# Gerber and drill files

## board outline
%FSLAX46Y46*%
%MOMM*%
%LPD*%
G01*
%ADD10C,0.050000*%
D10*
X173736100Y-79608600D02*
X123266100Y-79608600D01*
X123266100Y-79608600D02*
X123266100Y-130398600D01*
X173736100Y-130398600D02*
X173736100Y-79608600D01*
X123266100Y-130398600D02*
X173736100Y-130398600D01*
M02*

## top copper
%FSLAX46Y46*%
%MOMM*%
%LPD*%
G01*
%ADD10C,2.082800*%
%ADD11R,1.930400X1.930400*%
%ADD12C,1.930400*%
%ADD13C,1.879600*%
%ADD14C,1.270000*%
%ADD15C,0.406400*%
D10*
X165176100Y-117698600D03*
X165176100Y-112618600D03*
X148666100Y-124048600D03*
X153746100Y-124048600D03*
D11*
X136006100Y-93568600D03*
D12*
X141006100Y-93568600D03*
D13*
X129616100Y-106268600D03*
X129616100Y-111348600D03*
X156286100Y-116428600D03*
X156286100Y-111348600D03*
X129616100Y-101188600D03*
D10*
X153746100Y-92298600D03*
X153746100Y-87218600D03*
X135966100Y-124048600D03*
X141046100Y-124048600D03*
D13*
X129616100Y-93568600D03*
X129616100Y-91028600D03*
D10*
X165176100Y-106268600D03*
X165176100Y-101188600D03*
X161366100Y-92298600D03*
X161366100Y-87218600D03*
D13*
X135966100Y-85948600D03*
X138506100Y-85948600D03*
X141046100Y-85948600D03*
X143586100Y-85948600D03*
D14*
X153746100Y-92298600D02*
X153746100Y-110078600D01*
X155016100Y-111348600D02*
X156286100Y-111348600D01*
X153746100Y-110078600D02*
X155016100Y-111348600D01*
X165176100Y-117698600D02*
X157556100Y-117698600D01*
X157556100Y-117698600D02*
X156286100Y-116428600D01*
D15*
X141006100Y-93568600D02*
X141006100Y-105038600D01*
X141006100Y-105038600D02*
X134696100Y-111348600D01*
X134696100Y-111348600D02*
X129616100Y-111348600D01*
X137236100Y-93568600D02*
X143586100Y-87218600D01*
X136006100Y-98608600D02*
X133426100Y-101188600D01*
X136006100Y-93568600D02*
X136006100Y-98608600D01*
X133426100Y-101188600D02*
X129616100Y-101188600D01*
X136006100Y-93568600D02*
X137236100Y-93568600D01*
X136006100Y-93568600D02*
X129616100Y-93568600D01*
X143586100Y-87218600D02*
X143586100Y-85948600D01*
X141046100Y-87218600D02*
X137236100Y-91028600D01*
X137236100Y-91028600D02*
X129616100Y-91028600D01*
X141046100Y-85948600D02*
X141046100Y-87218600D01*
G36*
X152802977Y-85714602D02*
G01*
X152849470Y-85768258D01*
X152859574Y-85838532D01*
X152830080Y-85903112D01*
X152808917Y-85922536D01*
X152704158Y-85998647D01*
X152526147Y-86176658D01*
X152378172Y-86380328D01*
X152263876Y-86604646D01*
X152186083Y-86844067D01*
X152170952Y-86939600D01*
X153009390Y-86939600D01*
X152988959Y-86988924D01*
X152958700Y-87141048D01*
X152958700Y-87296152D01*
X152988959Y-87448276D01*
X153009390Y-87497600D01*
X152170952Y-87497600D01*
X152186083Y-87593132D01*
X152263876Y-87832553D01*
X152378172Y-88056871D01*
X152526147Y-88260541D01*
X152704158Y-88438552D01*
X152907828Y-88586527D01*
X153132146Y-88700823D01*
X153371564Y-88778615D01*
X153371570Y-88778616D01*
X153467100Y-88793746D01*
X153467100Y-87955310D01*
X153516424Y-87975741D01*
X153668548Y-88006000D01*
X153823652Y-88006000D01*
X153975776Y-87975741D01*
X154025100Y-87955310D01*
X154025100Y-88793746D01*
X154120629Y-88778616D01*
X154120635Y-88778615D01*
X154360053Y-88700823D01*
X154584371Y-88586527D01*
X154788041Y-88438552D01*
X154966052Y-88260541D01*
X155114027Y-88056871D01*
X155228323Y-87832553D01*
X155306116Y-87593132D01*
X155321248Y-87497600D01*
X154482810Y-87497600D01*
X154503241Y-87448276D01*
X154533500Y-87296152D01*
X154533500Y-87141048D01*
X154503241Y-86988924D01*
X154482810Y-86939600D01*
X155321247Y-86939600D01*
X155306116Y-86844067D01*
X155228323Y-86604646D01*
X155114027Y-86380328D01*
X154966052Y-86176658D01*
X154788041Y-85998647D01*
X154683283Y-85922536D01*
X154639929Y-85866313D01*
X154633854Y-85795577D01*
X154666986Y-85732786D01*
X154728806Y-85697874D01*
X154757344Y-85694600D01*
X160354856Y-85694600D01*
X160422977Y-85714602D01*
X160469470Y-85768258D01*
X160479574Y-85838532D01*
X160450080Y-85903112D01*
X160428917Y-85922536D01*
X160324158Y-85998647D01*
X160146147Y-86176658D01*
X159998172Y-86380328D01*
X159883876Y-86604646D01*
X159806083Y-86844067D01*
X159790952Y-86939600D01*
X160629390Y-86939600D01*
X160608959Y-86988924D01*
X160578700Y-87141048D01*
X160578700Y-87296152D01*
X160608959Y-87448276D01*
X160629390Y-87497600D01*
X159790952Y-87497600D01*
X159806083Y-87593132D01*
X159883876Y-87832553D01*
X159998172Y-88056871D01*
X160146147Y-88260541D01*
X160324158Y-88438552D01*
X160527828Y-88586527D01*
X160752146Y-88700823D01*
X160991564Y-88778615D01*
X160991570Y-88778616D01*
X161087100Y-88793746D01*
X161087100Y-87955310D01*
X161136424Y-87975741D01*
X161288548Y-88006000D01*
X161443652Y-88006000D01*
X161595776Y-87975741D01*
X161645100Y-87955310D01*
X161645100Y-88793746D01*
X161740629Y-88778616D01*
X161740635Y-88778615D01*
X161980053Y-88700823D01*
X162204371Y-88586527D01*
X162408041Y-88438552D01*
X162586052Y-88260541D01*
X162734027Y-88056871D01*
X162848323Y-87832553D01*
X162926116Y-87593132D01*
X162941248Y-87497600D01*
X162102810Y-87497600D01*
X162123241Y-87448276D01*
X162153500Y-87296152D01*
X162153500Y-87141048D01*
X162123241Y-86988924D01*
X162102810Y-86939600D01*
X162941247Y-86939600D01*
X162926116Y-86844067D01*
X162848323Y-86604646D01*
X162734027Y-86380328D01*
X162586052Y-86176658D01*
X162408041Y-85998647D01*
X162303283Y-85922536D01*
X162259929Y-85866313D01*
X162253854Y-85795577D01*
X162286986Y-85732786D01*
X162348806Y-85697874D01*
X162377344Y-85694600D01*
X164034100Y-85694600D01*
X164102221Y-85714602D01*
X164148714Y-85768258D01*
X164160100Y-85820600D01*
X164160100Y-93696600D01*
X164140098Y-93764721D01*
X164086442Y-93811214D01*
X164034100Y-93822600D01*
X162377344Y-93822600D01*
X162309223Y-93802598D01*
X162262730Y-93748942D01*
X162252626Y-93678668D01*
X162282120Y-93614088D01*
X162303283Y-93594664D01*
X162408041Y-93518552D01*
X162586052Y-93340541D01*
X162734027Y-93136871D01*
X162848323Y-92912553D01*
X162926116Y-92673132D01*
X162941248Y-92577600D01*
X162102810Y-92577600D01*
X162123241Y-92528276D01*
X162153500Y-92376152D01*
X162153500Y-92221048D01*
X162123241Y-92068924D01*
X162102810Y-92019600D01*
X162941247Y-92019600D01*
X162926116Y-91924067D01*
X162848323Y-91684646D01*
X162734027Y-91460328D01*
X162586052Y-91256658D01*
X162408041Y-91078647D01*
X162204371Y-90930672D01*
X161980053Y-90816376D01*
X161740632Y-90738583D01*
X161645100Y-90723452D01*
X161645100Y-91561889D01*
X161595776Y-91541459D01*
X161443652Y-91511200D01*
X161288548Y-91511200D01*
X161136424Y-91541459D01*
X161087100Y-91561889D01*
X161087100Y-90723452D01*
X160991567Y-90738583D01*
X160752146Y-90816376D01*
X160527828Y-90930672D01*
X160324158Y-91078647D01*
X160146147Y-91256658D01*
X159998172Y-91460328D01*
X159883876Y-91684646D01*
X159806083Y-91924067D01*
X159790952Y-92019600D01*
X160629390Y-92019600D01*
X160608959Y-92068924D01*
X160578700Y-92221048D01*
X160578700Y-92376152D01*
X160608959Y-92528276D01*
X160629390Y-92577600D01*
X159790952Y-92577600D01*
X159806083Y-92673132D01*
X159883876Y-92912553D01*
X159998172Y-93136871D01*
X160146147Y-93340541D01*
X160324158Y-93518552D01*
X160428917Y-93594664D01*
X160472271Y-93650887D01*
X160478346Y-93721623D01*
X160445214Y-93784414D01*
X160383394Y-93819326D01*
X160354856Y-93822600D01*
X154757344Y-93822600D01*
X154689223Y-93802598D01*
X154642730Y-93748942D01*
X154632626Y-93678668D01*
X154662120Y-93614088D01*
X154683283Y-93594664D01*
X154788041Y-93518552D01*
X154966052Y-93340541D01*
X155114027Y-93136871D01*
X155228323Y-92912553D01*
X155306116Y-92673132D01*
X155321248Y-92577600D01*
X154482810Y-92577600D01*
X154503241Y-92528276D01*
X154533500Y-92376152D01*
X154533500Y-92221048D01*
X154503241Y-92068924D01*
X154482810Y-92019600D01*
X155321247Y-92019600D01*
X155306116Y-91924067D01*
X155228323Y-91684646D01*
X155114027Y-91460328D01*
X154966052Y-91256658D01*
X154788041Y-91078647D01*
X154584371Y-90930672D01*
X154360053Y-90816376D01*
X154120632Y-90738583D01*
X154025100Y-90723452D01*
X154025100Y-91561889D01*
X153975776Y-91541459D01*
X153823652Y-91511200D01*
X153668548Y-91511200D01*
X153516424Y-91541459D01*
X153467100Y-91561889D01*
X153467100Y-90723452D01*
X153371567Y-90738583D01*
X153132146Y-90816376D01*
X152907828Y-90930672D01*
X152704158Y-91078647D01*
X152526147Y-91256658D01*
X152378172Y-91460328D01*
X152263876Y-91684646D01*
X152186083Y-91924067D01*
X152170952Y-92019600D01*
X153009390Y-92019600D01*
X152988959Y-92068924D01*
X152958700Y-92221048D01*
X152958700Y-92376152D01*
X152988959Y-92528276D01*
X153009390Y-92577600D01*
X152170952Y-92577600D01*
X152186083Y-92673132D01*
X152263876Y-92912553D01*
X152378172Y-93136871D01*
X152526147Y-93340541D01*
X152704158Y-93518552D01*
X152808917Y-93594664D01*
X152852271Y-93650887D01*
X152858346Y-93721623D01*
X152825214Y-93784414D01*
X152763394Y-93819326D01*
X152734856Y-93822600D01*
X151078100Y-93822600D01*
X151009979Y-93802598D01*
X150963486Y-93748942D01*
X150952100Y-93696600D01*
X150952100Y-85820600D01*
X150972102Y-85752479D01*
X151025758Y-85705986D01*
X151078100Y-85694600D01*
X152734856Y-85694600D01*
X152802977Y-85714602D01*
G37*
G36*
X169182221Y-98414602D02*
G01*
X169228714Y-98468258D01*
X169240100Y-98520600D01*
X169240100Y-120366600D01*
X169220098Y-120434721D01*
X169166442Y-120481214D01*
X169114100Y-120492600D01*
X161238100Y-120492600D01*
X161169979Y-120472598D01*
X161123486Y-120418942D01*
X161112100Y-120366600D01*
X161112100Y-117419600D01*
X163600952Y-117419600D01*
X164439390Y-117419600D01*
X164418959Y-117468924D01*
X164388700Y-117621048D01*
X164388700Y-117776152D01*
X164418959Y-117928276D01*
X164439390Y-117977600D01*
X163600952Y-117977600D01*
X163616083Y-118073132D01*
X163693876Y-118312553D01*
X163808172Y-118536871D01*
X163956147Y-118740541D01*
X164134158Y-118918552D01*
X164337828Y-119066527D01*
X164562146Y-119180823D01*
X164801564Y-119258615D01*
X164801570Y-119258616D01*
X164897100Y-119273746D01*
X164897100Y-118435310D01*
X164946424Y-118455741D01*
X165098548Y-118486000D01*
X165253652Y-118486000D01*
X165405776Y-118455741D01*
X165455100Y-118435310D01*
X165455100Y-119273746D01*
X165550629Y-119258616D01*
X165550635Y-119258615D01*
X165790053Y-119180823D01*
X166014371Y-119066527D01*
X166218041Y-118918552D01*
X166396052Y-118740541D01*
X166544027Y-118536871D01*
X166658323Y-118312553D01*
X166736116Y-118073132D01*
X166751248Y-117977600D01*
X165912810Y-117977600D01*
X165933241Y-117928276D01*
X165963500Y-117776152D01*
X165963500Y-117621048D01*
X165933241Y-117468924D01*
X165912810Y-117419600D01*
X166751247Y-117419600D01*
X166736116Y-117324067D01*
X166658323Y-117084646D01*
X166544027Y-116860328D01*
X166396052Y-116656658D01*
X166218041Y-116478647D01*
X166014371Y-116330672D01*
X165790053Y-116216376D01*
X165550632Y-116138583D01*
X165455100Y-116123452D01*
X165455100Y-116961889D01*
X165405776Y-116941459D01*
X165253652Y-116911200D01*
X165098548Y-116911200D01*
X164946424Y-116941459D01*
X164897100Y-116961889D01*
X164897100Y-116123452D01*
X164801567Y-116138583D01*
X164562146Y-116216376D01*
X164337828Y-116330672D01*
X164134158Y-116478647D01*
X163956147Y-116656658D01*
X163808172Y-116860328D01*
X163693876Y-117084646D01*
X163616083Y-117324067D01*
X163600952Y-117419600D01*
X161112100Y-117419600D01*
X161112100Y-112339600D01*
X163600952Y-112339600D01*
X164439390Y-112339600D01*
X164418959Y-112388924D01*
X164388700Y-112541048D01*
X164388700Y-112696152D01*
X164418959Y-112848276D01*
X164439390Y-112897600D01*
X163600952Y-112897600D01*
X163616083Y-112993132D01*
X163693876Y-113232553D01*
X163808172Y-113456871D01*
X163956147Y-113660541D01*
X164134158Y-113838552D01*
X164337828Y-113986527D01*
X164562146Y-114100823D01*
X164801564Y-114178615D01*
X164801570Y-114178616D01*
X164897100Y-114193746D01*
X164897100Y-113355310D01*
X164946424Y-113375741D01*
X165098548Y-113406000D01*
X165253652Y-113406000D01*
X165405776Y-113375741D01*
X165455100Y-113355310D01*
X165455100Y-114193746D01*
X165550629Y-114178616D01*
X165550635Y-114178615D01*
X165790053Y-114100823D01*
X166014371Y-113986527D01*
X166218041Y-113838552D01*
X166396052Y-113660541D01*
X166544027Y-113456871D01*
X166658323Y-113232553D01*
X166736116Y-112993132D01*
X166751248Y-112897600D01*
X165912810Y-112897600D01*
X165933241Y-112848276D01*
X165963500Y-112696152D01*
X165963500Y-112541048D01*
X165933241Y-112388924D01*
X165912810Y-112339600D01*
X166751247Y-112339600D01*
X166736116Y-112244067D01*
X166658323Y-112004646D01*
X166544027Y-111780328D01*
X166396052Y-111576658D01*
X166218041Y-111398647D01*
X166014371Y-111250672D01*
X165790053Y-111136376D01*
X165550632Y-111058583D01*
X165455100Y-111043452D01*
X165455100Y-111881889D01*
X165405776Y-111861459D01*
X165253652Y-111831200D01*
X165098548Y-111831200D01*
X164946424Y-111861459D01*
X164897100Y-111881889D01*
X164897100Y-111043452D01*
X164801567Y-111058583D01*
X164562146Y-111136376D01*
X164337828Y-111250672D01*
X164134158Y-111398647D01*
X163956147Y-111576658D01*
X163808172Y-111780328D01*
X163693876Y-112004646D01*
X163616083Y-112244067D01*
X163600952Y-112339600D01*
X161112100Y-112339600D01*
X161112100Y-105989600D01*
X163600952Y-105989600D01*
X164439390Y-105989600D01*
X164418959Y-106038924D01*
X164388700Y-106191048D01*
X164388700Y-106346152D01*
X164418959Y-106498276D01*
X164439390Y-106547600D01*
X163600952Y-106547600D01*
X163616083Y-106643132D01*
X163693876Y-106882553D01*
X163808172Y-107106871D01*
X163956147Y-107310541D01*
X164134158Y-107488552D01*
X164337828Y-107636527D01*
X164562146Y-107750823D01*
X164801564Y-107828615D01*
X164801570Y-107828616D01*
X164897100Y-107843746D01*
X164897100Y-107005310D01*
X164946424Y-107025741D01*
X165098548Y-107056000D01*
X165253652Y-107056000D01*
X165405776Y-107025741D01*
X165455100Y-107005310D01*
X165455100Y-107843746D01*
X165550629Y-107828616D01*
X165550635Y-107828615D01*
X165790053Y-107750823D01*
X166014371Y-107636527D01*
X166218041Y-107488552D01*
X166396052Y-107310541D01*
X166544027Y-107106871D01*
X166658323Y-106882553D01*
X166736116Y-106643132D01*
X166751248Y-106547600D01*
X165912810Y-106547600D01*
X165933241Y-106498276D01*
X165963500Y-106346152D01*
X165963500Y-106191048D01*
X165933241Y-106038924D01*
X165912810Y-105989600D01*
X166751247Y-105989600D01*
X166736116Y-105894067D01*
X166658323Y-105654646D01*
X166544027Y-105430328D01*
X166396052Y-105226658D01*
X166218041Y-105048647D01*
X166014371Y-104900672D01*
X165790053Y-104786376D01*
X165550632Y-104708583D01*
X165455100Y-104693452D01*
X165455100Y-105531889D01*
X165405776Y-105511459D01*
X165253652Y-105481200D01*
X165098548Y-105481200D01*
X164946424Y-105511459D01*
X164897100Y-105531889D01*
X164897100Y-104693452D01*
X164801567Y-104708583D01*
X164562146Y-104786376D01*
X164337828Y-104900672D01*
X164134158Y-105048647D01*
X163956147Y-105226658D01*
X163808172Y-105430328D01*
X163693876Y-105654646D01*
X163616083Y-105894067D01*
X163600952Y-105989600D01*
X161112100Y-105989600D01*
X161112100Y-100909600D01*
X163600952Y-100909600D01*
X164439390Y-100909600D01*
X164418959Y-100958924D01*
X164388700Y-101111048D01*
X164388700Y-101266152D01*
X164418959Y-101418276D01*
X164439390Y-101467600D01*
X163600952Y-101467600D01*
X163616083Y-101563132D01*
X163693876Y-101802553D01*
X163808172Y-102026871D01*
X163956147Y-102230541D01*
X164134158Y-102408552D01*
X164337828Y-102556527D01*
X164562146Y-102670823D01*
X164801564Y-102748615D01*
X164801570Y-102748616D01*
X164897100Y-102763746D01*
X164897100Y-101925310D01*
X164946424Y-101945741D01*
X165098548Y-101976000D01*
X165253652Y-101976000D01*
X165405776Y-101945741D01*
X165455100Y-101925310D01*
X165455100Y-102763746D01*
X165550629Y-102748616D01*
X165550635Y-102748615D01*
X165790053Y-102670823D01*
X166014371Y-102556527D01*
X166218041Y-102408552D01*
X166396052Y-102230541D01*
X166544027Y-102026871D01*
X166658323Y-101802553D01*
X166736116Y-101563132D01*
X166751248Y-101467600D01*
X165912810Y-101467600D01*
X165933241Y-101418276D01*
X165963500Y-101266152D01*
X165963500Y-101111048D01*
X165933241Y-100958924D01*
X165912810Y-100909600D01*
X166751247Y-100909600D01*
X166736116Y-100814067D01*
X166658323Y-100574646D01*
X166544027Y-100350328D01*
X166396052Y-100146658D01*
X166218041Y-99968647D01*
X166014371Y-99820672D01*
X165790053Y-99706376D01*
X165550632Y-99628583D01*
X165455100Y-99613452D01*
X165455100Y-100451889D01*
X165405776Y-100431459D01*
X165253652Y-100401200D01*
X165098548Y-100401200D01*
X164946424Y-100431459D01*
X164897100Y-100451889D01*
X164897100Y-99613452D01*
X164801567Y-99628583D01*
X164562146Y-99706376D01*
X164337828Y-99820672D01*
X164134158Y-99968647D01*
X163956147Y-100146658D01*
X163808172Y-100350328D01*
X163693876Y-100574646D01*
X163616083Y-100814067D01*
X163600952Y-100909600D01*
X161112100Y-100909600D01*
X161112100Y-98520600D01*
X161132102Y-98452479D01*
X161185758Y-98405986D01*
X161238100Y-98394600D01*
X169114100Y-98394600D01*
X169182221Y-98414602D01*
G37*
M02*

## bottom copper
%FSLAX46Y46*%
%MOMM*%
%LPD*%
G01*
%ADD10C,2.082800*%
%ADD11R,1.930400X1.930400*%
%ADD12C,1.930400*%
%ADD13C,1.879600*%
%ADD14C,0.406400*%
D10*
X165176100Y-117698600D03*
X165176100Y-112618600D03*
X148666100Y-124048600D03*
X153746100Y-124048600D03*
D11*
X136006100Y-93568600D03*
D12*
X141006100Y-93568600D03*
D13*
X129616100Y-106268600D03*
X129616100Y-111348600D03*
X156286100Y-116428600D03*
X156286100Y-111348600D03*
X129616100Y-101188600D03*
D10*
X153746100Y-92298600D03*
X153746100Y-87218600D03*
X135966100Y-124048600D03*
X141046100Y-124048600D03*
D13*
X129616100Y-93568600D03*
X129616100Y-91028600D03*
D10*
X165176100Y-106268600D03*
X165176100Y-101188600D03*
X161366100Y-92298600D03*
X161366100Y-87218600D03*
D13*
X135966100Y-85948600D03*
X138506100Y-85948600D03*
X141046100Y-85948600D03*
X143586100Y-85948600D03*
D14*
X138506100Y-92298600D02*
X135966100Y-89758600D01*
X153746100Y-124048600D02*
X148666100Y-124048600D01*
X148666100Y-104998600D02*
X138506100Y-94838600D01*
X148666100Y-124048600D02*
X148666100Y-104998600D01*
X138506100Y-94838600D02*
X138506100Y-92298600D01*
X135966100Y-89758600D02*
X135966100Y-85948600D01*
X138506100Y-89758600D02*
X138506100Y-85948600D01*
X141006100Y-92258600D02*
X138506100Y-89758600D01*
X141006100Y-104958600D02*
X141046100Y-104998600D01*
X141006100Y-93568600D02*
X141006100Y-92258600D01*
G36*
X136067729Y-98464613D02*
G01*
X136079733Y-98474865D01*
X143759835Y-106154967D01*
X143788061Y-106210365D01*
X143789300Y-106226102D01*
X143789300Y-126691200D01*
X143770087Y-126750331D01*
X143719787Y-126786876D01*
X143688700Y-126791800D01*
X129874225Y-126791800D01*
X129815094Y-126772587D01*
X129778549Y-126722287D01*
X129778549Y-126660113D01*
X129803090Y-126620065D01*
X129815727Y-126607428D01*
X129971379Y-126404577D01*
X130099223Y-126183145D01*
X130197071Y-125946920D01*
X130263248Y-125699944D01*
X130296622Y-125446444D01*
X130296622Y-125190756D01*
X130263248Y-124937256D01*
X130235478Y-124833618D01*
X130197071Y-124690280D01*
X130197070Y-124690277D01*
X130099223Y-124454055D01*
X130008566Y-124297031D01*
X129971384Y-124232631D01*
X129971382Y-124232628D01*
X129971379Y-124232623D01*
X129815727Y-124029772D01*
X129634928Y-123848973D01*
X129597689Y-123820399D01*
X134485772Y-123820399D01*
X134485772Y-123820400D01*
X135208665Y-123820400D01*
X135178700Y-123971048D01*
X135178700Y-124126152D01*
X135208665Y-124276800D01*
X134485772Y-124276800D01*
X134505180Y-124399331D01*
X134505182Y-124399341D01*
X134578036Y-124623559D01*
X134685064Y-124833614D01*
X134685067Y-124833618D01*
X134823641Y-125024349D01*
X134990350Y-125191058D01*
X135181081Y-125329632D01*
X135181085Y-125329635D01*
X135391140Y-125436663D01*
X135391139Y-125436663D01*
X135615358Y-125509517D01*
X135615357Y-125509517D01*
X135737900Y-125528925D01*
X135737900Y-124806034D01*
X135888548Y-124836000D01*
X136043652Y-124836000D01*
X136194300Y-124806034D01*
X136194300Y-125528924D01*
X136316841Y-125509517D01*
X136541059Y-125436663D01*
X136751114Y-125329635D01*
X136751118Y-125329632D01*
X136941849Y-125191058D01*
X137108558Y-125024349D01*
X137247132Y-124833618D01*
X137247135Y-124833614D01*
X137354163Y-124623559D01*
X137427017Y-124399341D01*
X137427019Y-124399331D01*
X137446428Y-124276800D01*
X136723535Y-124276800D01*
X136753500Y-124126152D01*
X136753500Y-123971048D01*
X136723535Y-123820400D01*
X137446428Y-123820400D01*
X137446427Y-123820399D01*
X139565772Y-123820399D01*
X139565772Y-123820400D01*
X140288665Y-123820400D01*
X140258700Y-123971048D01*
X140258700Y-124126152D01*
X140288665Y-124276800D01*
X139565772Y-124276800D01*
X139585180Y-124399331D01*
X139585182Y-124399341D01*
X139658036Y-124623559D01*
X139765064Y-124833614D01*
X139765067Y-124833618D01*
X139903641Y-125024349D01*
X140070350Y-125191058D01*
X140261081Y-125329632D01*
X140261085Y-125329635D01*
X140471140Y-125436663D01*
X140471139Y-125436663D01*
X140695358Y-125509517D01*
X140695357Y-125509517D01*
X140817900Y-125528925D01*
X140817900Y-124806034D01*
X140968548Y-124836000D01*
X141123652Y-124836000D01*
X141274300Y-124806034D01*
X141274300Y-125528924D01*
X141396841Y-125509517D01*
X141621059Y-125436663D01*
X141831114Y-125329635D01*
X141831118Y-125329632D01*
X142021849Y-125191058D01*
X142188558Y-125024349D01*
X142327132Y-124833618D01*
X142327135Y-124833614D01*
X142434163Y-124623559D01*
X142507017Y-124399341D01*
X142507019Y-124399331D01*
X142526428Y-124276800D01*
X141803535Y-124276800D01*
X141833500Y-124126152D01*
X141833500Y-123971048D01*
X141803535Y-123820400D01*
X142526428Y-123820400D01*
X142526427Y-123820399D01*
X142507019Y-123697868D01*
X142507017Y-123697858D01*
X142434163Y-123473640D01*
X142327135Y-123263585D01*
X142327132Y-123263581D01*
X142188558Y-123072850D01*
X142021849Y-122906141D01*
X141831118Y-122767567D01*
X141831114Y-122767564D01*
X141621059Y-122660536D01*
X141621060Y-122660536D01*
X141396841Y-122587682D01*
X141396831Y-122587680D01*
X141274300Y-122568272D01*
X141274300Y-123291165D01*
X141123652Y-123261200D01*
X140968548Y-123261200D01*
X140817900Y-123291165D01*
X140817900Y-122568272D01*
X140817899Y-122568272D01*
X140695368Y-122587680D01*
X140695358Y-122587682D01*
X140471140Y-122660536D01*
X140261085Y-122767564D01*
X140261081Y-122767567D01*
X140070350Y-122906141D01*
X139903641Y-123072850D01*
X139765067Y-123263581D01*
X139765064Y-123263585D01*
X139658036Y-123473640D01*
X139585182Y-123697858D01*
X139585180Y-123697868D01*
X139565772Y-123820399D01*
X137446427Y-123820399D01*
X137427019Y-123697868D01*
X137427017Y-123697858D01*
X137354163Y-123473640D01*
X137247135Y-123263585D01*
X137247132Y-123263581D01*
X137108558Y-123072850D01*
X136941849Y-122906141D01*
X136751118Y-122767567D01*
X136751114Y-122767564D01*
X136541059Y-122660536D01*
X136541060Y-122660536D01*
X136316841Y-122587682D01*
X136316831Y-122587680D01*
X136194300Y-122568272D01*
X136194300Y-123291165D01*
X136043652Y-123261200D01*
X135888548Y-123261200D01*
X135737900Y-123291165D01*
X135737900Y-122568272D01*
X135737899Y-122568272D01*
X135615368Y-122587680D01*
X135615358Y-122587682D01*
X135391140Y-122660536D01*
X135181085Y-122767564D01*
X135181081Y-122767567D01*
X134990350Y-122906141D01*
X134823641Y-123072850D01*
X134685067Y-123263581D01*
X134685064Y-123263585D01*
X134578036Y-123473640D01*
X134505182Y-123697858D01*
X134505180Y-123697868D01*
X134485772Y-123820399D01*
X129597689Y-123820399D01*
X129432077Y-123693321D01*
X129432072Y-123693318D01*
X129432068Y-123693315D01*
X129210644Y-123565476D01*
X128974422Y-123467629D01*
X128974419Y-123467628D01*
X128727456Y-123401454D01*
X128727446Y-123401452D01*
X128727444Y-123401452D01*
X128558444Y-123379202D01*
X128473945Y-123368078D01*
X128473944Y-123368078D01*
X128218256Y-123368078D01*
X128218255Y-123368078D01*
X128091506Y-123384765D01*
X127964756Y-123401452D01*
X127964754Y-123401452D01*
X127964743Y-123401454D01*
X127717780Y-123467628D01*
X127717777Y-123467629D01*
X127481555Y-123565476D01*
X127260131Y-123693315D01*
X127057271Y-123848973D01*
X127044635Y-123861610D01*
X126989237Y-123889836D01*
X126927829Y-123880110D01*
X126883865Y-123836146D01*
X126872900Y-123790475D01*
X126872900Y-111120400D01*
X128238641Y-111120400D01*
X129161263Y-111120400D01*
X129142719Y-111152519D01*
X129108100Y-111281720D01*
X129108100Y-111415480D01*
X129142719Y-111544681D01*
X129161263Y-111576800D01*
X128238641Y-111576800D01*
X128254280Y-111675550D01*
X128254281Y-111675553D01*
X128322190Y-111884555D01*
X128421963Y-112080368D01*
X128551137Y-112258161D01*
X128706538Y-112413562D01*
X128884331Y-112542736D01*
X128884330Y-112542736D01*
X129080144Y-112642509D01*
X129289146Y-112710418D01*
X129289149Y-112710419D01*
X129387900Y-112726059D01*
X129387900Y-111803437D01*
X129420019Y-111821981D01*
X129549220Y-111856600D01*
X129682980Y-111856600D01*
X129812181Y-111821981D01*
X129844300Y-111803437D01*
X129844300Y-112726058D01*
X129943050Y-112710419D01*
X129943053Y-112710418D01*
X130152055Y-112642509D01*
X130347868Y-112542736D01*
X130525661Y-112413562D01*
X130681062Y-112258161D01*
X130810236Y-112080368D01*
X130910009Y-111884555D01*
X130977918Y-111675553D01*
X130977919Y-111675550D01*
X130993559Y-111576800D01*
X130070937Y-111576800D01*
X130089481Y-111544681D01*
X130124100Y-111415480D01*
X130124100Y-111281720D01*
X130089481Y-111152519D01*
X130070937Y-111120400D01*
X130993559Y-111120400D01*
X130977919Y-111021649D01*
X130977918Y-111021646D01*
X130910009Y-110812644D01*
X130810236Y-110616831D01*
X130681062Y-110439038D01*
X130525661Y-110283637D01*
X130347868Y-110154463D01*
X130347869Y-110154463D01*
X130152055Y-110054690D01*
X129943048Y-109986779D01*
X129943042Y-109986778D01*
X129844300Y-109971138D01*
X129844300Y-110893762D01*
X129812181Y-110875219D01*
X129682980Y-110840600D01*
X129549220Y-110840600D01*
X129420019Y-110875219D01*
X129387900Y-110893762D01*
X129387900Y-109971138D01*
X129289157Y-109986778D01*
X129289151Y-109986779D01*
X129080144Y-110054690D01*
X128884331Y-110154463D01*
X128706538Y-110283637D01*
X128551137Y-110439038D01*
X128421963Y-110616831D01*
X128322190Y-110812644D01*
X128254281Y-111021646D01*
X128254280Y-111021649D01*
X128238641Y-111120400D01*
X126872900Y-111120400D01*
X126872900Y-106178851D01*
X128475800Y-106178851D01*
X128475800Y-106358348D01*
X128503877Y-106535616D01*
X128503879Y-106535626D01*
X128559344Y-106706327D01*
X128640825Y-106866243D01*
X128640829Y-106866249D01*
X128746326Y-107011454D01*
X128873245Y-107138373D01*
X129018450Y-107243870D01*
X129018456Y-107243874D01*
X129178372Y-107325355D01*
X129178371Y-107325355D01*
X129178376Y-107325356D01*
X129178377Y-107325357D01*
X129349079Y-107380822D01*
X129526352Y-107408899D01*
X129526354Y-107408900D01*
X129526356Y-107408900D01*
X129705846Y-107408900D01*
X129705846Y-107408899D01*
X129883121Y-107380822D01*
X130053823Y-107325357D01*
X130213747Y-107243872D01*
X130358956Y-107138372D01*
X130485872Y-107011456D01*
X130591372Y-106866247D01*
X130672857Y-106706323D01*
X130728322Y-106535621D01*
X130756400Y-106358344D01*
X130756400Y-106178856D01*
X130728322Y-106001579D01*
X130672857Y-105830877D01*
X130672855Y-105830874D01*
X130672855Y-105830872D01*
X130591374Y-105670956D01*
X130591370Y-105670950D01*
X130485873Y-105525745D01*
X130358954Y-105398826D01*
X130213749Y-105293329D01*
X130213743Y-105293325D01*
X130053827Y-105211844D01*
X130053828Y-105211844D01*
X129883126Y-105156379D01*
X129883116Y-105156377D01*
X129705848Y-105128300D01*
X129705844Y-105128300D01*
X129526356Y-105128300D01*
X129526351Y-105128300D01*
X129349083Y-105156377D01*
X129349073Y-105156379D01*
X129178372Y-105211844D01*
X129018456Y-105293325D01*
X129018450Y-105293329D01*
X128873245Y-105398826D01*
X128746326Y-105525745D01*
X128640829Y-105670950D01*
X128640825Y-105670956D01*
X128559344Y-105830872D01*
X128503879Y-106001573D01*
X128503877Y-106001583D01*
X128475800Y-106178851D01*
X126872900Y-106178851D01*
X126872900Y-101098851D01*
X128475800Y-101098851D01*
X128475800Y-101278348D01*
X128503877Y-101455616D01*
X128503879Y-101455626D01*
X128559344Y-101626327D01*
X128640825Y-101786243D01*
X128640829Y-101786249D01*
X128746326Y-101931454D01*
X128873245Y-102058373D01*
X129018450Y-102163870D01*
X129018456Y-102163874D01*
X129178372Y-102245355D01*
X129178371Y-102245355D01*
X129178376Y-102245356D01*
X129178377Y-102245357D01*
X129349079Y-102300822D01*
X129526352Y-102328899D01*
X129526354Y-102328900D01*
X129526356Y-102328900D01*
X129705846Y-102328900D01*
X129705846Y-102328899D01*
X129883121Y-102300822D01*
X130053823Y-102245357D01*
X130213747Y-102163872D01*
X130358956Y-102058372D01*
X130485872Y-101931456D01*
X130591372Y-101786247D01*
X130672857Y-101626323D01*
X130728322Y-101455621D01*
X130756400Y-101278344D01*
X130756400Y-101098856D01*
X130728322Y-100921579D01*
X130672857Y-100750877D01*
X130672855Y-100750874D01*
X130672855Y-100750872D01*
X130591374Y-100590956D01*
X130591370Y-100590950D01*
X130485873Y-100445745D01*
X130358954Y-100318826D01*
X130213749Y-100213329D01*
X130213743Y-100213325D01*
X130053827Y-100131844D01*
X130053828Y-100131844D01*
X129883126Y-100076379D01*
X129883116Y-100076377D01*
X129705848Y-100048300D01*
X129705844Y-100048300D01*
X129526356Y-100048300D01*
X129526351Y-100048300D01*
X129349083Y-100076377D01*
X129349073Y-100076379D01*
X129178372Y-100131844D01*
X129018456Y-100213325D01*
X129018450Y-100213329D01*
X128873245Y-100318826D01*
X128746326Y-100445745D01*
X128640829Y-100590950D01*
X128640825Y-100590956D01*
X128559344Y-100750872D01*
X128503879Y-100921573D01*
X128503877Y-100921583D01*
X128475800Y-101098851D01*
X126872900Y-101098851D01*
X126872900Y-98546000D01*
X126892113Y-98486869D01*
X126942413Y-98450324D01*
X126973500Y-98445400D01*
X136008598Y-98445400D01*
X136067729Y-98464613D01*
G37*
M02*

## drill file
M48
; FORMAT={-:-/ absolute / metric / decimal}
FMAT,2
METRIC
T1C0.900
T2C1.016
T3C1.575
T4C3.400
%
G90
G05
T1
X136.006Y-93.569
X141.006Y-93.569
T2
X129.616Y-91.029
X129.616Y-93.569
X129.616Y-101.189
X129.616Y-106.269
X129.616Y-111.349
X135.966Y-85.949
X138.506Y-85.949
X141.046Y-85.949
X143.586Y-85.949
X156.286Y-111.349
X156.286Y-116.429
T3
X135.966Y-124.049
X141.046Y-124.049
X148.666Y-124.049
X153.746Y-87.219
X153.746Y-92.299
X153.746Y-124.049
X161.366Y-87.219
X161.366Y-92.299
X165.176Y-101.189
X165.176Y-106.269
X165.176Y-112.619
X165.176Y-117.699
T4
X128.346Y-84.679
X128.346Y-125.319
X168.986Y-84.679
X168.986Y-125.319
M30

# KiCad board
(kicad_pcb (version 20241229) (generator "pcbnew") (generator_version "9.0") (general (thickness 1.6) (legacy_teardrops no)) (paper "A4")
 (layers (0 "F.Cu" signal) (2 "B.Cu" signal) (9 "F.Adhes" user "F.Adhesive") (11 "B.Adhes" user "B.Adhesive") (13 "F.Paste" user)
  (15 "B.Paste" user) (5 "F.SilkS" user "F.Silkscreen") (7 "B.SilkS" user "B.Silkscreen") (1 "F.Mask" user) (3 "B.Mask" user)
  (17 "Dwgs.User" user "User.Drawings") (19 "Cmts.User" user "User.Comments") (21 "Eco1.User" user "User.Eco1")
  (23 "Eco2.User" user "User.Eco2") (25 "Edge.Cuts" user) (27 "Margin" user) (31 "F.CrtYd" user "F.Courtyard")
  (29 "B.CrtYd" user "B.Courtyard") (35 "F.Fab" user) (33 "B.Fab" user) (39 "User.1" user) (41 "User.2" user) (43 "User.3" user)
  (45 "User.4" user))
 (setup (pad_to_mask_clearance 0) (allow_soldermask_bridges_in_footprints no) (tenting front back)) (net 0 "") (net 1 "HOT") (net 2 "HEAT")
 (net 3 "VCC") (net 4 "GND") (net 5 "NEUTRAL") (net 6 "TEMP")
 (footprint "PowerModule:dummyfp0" (layer "F.Cu") (at 168.9861 125.3186)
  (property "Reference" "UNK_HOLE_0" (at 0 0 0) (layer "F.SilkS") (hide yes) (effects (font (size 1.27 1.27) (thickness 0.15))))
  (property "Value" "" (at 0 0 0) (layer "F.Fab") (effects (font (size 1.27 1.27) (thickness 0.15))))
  (pad "" np_thru_hole circle (at 0 0) (size 3.400043 3.400043) (drill 3.400043) (layers "*.Cu" "*.Mask")))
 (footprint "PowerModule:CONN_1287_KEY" (layer "F.Cu") (at 165.1761 117.6986 90)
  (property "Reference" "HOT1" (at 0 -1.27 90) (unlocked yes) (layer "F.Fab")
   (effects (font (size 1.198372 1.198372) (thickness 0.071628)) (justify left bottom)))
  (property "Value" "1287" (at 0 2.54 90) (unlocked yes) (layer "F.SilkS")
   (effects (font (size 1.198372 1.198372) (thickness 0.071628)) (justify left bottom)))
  (pad "1" thru_hole circle (at 0 0 90) (size 2.0828 2.0828) (drill 1.5748) (layers "*.Cu" "*.Mask") (remove_unused_layers no) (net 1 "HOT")
   (solder_mask_margin 0.0635) (thermal_bridge_angle 0))
  (pad "2" thru_hole circle (at 5.08 0 90) (size 2.0828 2.0828) (drill 1.5748) (layers "*.Cu" "*.Mask") (remove_unused_layers no)
   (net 1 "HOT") (solder_mask_margin 0.0635) (thermal_bridge_angle 0)))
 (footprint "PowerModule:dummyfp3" (layer "F.Cu") (at 128.3461 84.6786)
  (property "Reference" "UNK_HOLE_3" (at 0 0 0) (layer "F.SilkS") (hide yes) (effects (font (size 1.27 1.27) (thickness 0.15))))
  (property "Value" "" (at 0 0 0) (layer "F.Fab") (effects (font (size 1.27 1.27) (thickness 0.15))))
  (pad "" np_thru_hole circle (at 0 0) (size 3.400043 3.400043) (drill 3.400043) (layers "*.Cu" "*.Mask")))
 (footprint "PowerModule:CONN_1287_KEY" (layer "F.Cu") (at 148.6661 124.0486)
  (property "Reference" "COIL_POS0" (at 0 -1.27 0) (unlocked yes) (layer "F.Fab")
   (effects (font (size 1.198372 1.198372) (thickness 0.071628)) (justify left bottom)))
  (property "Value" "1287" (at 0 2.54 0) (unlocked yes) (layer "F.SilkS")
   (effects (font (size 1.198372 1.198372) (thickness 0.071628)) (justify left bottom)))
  (pad "1" thru_hole circle (at 0 0) (size 2.0828 2.0828) (drill 1.5748) (layers "*.Cu" "*.Mask") (remove_unused_layers no) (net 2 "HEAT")
   (solder_mask_margin 0.0635) (thermal_bridge_angle 0))
  (pad "2" thru_hole circle (at 5.08 0) (size 2.0828 2.0828) (drill 1.5748) (layers "*.Cu" "*.Mask") (remove_unused_layers no)
   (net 2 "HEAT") (solder_mask_margin 0.0635) (thermal_bridge_angle 0)))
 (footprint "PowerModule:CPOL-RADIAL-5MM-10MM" (layer "F.Cu") (at 138.5061 93.5686 180)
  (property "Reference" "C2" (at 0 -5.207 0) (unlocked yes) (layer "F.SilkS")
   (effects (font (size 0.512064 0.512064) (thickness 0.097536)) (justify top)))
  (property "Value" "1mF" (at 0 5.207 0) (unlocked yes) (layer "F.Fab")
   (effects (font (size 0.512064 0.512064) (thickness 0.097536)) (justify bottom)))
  (pad "+" thru_hole rect (at 2.5 0 180) (size 1.9304 1.9304) (drill 0.9) (layers "*.Cu" "*.Mask") (remove_unused_layers no) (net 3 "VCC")
   (solder_mask_margin 0.0635) (thermal_bridge_angle 0))
  (pad "-" thru_hole circle (at -2.5 0 180) (size 1.9304 1.9304) (drill 0.9) (layers "*.Cu" "*.Mask") (remove_unused_layers no)
   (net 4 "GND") (solder_mask_margin 0.0635) (thermal_bridge_angle 0)))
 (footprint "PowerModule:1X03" (layer "F.Cu") (at 156.2861 116.4286 90)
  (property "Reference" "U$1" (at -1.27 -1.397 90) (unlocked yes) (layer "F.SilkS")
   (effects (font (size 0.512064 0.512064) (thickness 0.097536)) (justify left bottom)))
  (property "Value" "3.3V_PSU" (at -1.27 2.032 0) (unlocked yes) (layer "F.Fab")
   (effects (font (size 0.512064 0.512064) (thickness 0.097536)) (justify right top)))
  (pad "5" thru_hole circle (at 10.16 -26.67 180) (size 1.8796 1.8796) (drill 1.016) (layers "*.Cu" "*.Mask") (remove_unused_layers no)
   (solder_mask_margin 0.0635) (thermal_bridge_angle 0))
  (pad "GND" thru_hole circle (at 5.08 -26.67 180) (size 1.8796 1.8796) (drill 1.016) (layers "*.Cu" "*.Mask") (remove_unused_layers no)
   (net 4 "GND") (solder_mask_margin 0.0635) (thermal_bridge_angle 0))
  (pad "HOT" thru_hole circle (at 0 0 180) (size 1.8796 1.8796) (drill 1.016) (layers "*.Cu" "*.Mask") (remove_unused_layers no)
   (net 1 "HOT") (solder_mask_margin 0.0635) (thermal_bridge_angle 0))
  (pad "NEUTRAL" thru_hole circle (at 5.08 0 180) (size 1.8796 1.8796) (drill 1.016) (layers "*.Cu" "*.Mask") (remove_unused_layers no)
   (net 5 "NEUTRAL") (solder_mask_margin 0.0635) (thermal_bridge_angle 0))
  (pad "VCC" thru_hole circle (at 15.24 -26.67 180) (size 1.8796 1.8796) (drill 1.016) (layers "*.Cu" "*.Mask") (remove_unused_layers no)
   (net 3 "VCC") (solder_mask_margin 0.0635) (thermal_bridge_angle 0)))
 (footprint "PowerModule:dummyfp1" (layer "F.Cu") (at 128.3461 125.3186)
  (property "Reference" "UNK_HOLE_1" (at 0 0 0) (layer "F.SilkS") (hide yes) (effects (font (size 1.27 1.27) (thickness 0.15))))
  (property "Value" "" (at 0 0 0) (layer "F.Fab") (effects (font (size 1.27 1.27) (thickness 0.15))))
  (pad "" np_thru_hole circle (at 0 0) (size 3.400043 3.400043) (drill 3.400043) (layers "*.Cu" "*.Mask")))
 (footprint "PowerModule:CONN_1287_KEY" (layer "F.Cu") (at 153.7461 92.2986 90)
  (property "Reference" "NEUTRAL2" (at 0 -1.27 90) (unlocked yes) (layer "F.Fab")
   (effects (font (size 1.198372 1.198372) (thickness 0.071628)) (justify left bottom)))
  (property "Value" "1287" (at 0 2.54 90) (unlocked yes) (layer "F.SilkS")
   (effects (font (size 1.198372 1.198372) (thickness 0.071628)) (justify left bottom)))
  (pad "1" thru_hole circle (at 0 0 90) (size 2.0828 2.0828) (drill 1.5748) (layers "*.Cu" "*.Mask") (remove_unused_layers no)
   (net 5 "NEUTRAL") (solder_mask_margin 0.0635) (thermal_bridge_angle 0))
  (pad "2" thru_hole circle (at 5.08 0 90) (size 2.0828 2.0828) (drill 1.5748) (layers "*.Cu" "*.Mask") (remove_unused_layers no)
   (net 5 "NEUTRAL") (solder_mask_margin 0.0635) (thermal_bridge_angle 0)))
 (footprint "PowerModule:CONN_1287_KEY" (layer "F.Cu") (at 135.9661 124.0486)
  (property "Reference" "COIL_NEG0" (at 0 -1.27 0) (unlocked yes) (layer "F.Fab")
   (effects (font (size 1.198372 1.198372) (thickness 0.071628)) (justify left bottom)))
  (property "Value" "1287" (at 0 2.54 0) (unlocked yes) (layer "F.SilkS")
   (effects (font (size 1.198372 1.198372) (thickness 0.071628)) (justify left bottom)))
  (pad "1" thru_hole circle (at 0 0) (size 2.0828 2.0828) (drill 1.5748) (layers "*.Cu" "*.Mask") (remove_unused_layers no) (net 4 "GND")
   (solder_mask_margin 0.0635) (thermal_bridge_angle 0))
  (pad "2" thru_hole circle (at 5.08 0) (size 2.0828 2.0828) (drill 1.5748) (layers "*.Cu" "*.Mask") (remove_unused_layers no) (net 4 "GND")
   (solder_mask_margin 0.0635) (thermal_bridge_angle 0)))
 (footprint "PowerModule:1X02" (layer "F.Cu") (at 129.6161 93.5686 90)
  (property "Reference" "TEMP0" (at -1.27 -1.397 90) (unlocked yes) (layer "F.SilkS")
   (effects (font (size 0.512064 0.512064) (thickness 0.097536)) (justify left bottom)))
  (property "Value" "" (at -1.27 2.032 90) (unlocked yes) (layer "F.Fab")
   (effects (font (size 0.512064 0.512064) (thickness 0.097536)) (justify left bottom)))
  (pad "1" thru_hole circle (at 0 0 180) (size 1.8796 1.8796) (drill 1.016) (layers "*.Cu" "*.Mask") (remove_unused_layers no) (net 3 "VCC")
   (solder_mask_margin 0.0635) (thermal_bridge_angle 0))
  (pad "2" thru_hole circle (at 2.54 0 180) (size 1.8796 1.8796) (drill 1.016) (layers "*.Cu" "*.Mask") (remove_unused_layers no)
   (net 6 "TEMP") (solder_mask_margin 0.0635) (thermal_bridge_angle 0)))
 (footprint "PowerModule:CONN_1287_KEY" (layer "F.Cu") (at 165.1761 106.2686 90)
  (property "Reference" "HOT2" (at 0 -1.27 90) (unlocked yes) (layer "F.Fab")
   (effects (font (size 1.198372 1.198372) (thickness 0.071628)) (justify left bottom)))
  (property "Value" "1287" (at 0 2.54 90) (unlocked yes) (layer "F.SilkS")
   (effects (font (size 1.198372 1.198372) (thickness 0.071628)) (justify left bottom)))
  (pad "1" thru_hole circle (at 0 0 90) (size 2.0828 2.0828) (drill 1.5748) (layers "*.Cu" "*.Mask") (remove_unused_layers no) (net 1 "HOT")
   (solder_mask_margin 0.0635) (thermal_bridge_angle 0))
  (pad "2" thru_hole circle (at 5.08 0 90) (size 2.0828 2.0828) (drill 1.5748) (layers "*.Cu" "*.Mask") (remove_unused_layers no)
   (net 1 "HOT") (solder_mask_margin 0.0635) (thermal_bridge_angle 0)))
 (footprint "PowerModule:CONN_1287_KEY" (layer "F.Cu") (at 161.3661 92.2986 90)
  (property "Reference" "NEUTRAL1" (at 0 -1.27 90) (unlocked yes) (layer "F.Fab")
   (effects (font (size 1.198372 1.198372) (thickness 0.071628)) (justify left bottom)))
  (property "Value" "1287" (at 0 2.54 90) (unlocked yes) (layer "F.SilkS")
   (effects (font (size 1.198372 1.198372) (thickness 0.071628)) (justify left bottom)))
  (pad "1" thru_hole circle (at 0 0 90) (size 2.0828 2.0828) (drill 1.5748) (layers "*.Cu" "*.Mask") (remove_unused_layers no)
   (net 5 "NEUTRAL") (solder_mask_margin 0.0635) (thermal_bridge_angle 0))
  (pad "2" thru_hole circle (at 5.08 0 90) (size 2.0828 2.0828) (drill 1.5748) (layers "*.Cu" "*.Mask") (remove_unused_layers no)
   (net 5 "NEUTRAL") (solder_mask_margin 0.0635) (thermal_bridge_angle 0)))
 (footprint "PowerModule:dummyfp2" (layer "F.Cu") (at 168.9861 84.6786)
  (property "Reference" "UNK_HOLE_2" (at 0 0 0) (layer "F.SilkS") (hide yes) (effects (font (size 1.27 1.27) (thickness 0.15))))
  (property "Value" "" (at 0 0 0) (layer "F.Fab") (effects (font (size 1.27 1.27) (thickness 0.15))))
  (pad "" np_thru_hole circle (at 0 0) (size 3.400043 3.400043) (drill 3.400043) (layers "*.Cu" "*.Mask")))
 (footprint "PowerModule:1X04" (layer "F.Cu") (at 135.9661 85.9486)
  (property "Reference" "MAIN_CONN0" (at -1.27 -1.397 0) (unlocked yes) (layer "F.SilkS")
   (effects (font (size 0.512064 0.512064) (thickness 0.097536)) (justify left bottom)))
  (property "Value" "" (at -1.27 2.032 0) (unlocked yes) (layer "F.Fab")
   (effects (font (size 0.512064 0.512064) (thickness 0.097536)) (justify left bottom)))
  (pad "1" thru_hole circle (at 0 0 90) (size 1.8796 1.8796) (drill 1.016) (layers "*.Cu" "*.Mask") (remove_unused_layers no) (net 2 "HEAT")
   (solder_mask_margin 0.0635) (thermal_bridge_angle 0))
  (pad "2" thru_hole circle (at 2.54 0 90) (size 1.8796 1.8796) (drill 1.016) (layers "*.Cu" "*.Mask") (remove_unused_layers no)
   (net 4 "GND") (solder_mask_margin 0.0635) (thermal_bridge_angle 0))
  (pad "3" thru_hole circle (at 5.08 0 90) (size 1.8796 1.8796) (drill 1.016) (layers "*.Cu" "*.Mask") (remove_unused_layers no)
   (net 6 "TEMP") (solder_mask_margin 0.0635) (thermal_bridge_angle 0))
  (pad "4" thru_hole circle (at 7.62 0 90) (size 1.8796 1.8796) (drill 1.016) (layers "*.Cu" "*.Mask") (remove_unused_layers no)
   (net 3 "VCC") (solder_mask_margin 0.0635) (thermal_bridge_angle 0)))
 (gr_line (start 173.7361 79.6086) (end 123.2661 79.6086) (stroke (width 0.05) (type solid)) (layer "Edge.Cuts"))
 (gr_line (start 123.2661 79.6086) (end 123.2661 130.3986) (stroke (width 0.05) (type solid)) (layer "Edge.Cuts"))
 (gr_line (start 173.7361 130.3986) (end 173.7361 79.6086) (stroke (width 0.05) (type solid)) (layer "Edge.Cuts"))
 (gr_line (start 123.2661 130.3986) (end 173.7361 130.3986) (stroke (width 0.05) (type solid)) (layer "Edge.Cuts"))
 (segment (start 153.7461 92.2986) (end 153.7461 110.0786) (width 1.27) (layer "F.Cu") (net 5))
 (segment (start 155.0161 111.3486) (end 156.2861 111.3486) (width 1.27) (layer "F.Cu") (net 5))
 (segment (start 153.7461 110.0786) (end 155.0161 111.3486) (width 1.27) (layer "F.Cu") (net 5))
 (segment (start 165.1761 117.6986) (end 157.5561 117.6986) (width 1.27) (layer "F.Cu") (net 1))
 (segment (start 157.5561 117.6986) (end 156.2861 116.4286) (width 1.27) (layer "F.Cu") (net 1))
 (segment (start 138.5061 92.2986) (end 135.9661 89.7586) (width 0.4064) (layer "B.Cu") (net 2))
 (segment (start 153.7461 124.0486) (end 148.6661 124.0486) (width 0.4064) (layer "B.Cu") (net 2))
 (segment (start 148.6661 104.9986) (end 138.5061 94.8386) (width 0.4064) (layer "B.Cu") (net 2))
 (segment (start 148.6661 124.0486) (end 148.6661 104.9986) (width 0.4064) (layer "B.Cu") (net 2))
 (segment (start 138.5061 94.8386) (end 138.5061 92.2986) (width 0.4064) (layer "B.Cu") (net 2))
 (segment (start 135.9661 89.7586) (end 135.9661 85.9486) (width 0.4064) (layer "B.Cu") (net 2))
 (segment (start 141.0061 93.5686) (end 141.0061 105.0386) (width 0.4064) (layer "F.Cu") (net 4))
 (segment (start 141.0061 105.0386) (end 134.6961 111.3486) (width 0.4064) (layer "F.Cu") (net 4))
 (segment (start 134.6961 111.3486) (end 129.6161 111.3486) (width 0.4064) (layer "F.Cu") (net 4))
 (segment (start 138.5061 89.7586) (end 138.5061 85.9486) (width 0.4064) (layer "B.Cu") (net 4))
 (segment (start 141.0061 92.2586) (end 138.5061 89.7586) (width 0.4064) (layer "B.Cu") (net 4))
 (segment (start 141.0061 104.9586) (end 141.0461 104.9986) (width 0.4064) (layer "B.Cu") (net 4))
 (segment (start 141.0061 93.5686) (end 141.0061 92.2586) (width 0.4064) (layer "B.Cu") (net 4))
 (segment (start 137.2361 93.5686) (end 143.5861 87.2186) (width 0.4064) (layer "F.Cu") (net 3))
 (segment (start 136.0061 98.6086) (end 133.4261 101.1886) (width 0.4064) (layer "F.Cu") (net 3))
 (segment (start 136.0061 93.5686) (end 136.0061 98.6086) (width 0.4064) (layer "F.Cu") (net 3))
 (segment (start 133.4261 101.1886) (end 129.6161 101.1886) (width 0.4064) (layer "F.Cu") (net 3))
 (segment (start 136.0061 93.5686) (end 137.2361 93.5686) (width 0.4064) (layer "F.Cu") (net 3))
 (segment (start 136.0061 93.5686) (end 129.6161 93.5686) (width 0.4064) (layer "F.Cu") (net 3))
 (segment (start 143.5861 87.2186) (end 143.5861 85.9486) (width 0.4064) (layer "F.Cu") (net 3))
 (segment (start 141.0461 87.2186) (end 137.2361 91.0286) (width 0.4064) (layer "F.Cu") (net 6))
 (segment (start 137.2361 91.0286) (end 129.6161 91.0286) (width 0.4064) (layer "F.Cu") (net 6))
 (segment (start 141.0461 85.9486) (end 141.0461 87.2186) (width 0.4064) (layer "F.Cu") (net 6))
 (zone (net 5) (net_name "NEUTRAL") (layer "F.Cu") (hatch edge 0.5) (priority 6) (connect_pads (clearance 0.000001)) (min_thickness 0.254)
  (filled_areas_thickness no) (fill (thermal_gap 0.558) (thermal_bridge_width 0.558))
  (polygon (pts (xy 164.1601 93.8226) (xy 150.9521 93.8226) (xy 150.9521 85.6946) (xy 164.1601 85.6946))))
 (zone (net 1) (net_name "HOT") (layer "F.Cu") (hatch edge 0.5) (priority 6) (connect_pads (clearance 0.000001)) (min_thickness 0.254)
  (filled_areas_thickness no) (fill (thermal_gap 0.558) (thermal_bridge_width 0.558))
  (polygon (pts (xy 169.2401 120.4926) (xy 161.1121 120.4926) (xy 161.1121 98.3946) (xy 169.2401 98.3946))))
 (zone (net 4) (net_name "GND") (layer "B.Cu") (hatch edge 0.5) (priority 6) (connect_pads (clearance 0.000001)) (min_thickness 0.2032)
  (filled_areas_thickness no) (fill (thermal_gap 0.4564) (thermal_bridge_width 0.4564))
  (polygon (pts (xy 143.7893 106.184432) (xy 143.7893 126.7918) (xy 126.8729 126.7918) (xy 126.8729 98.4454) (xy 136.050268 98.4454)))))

